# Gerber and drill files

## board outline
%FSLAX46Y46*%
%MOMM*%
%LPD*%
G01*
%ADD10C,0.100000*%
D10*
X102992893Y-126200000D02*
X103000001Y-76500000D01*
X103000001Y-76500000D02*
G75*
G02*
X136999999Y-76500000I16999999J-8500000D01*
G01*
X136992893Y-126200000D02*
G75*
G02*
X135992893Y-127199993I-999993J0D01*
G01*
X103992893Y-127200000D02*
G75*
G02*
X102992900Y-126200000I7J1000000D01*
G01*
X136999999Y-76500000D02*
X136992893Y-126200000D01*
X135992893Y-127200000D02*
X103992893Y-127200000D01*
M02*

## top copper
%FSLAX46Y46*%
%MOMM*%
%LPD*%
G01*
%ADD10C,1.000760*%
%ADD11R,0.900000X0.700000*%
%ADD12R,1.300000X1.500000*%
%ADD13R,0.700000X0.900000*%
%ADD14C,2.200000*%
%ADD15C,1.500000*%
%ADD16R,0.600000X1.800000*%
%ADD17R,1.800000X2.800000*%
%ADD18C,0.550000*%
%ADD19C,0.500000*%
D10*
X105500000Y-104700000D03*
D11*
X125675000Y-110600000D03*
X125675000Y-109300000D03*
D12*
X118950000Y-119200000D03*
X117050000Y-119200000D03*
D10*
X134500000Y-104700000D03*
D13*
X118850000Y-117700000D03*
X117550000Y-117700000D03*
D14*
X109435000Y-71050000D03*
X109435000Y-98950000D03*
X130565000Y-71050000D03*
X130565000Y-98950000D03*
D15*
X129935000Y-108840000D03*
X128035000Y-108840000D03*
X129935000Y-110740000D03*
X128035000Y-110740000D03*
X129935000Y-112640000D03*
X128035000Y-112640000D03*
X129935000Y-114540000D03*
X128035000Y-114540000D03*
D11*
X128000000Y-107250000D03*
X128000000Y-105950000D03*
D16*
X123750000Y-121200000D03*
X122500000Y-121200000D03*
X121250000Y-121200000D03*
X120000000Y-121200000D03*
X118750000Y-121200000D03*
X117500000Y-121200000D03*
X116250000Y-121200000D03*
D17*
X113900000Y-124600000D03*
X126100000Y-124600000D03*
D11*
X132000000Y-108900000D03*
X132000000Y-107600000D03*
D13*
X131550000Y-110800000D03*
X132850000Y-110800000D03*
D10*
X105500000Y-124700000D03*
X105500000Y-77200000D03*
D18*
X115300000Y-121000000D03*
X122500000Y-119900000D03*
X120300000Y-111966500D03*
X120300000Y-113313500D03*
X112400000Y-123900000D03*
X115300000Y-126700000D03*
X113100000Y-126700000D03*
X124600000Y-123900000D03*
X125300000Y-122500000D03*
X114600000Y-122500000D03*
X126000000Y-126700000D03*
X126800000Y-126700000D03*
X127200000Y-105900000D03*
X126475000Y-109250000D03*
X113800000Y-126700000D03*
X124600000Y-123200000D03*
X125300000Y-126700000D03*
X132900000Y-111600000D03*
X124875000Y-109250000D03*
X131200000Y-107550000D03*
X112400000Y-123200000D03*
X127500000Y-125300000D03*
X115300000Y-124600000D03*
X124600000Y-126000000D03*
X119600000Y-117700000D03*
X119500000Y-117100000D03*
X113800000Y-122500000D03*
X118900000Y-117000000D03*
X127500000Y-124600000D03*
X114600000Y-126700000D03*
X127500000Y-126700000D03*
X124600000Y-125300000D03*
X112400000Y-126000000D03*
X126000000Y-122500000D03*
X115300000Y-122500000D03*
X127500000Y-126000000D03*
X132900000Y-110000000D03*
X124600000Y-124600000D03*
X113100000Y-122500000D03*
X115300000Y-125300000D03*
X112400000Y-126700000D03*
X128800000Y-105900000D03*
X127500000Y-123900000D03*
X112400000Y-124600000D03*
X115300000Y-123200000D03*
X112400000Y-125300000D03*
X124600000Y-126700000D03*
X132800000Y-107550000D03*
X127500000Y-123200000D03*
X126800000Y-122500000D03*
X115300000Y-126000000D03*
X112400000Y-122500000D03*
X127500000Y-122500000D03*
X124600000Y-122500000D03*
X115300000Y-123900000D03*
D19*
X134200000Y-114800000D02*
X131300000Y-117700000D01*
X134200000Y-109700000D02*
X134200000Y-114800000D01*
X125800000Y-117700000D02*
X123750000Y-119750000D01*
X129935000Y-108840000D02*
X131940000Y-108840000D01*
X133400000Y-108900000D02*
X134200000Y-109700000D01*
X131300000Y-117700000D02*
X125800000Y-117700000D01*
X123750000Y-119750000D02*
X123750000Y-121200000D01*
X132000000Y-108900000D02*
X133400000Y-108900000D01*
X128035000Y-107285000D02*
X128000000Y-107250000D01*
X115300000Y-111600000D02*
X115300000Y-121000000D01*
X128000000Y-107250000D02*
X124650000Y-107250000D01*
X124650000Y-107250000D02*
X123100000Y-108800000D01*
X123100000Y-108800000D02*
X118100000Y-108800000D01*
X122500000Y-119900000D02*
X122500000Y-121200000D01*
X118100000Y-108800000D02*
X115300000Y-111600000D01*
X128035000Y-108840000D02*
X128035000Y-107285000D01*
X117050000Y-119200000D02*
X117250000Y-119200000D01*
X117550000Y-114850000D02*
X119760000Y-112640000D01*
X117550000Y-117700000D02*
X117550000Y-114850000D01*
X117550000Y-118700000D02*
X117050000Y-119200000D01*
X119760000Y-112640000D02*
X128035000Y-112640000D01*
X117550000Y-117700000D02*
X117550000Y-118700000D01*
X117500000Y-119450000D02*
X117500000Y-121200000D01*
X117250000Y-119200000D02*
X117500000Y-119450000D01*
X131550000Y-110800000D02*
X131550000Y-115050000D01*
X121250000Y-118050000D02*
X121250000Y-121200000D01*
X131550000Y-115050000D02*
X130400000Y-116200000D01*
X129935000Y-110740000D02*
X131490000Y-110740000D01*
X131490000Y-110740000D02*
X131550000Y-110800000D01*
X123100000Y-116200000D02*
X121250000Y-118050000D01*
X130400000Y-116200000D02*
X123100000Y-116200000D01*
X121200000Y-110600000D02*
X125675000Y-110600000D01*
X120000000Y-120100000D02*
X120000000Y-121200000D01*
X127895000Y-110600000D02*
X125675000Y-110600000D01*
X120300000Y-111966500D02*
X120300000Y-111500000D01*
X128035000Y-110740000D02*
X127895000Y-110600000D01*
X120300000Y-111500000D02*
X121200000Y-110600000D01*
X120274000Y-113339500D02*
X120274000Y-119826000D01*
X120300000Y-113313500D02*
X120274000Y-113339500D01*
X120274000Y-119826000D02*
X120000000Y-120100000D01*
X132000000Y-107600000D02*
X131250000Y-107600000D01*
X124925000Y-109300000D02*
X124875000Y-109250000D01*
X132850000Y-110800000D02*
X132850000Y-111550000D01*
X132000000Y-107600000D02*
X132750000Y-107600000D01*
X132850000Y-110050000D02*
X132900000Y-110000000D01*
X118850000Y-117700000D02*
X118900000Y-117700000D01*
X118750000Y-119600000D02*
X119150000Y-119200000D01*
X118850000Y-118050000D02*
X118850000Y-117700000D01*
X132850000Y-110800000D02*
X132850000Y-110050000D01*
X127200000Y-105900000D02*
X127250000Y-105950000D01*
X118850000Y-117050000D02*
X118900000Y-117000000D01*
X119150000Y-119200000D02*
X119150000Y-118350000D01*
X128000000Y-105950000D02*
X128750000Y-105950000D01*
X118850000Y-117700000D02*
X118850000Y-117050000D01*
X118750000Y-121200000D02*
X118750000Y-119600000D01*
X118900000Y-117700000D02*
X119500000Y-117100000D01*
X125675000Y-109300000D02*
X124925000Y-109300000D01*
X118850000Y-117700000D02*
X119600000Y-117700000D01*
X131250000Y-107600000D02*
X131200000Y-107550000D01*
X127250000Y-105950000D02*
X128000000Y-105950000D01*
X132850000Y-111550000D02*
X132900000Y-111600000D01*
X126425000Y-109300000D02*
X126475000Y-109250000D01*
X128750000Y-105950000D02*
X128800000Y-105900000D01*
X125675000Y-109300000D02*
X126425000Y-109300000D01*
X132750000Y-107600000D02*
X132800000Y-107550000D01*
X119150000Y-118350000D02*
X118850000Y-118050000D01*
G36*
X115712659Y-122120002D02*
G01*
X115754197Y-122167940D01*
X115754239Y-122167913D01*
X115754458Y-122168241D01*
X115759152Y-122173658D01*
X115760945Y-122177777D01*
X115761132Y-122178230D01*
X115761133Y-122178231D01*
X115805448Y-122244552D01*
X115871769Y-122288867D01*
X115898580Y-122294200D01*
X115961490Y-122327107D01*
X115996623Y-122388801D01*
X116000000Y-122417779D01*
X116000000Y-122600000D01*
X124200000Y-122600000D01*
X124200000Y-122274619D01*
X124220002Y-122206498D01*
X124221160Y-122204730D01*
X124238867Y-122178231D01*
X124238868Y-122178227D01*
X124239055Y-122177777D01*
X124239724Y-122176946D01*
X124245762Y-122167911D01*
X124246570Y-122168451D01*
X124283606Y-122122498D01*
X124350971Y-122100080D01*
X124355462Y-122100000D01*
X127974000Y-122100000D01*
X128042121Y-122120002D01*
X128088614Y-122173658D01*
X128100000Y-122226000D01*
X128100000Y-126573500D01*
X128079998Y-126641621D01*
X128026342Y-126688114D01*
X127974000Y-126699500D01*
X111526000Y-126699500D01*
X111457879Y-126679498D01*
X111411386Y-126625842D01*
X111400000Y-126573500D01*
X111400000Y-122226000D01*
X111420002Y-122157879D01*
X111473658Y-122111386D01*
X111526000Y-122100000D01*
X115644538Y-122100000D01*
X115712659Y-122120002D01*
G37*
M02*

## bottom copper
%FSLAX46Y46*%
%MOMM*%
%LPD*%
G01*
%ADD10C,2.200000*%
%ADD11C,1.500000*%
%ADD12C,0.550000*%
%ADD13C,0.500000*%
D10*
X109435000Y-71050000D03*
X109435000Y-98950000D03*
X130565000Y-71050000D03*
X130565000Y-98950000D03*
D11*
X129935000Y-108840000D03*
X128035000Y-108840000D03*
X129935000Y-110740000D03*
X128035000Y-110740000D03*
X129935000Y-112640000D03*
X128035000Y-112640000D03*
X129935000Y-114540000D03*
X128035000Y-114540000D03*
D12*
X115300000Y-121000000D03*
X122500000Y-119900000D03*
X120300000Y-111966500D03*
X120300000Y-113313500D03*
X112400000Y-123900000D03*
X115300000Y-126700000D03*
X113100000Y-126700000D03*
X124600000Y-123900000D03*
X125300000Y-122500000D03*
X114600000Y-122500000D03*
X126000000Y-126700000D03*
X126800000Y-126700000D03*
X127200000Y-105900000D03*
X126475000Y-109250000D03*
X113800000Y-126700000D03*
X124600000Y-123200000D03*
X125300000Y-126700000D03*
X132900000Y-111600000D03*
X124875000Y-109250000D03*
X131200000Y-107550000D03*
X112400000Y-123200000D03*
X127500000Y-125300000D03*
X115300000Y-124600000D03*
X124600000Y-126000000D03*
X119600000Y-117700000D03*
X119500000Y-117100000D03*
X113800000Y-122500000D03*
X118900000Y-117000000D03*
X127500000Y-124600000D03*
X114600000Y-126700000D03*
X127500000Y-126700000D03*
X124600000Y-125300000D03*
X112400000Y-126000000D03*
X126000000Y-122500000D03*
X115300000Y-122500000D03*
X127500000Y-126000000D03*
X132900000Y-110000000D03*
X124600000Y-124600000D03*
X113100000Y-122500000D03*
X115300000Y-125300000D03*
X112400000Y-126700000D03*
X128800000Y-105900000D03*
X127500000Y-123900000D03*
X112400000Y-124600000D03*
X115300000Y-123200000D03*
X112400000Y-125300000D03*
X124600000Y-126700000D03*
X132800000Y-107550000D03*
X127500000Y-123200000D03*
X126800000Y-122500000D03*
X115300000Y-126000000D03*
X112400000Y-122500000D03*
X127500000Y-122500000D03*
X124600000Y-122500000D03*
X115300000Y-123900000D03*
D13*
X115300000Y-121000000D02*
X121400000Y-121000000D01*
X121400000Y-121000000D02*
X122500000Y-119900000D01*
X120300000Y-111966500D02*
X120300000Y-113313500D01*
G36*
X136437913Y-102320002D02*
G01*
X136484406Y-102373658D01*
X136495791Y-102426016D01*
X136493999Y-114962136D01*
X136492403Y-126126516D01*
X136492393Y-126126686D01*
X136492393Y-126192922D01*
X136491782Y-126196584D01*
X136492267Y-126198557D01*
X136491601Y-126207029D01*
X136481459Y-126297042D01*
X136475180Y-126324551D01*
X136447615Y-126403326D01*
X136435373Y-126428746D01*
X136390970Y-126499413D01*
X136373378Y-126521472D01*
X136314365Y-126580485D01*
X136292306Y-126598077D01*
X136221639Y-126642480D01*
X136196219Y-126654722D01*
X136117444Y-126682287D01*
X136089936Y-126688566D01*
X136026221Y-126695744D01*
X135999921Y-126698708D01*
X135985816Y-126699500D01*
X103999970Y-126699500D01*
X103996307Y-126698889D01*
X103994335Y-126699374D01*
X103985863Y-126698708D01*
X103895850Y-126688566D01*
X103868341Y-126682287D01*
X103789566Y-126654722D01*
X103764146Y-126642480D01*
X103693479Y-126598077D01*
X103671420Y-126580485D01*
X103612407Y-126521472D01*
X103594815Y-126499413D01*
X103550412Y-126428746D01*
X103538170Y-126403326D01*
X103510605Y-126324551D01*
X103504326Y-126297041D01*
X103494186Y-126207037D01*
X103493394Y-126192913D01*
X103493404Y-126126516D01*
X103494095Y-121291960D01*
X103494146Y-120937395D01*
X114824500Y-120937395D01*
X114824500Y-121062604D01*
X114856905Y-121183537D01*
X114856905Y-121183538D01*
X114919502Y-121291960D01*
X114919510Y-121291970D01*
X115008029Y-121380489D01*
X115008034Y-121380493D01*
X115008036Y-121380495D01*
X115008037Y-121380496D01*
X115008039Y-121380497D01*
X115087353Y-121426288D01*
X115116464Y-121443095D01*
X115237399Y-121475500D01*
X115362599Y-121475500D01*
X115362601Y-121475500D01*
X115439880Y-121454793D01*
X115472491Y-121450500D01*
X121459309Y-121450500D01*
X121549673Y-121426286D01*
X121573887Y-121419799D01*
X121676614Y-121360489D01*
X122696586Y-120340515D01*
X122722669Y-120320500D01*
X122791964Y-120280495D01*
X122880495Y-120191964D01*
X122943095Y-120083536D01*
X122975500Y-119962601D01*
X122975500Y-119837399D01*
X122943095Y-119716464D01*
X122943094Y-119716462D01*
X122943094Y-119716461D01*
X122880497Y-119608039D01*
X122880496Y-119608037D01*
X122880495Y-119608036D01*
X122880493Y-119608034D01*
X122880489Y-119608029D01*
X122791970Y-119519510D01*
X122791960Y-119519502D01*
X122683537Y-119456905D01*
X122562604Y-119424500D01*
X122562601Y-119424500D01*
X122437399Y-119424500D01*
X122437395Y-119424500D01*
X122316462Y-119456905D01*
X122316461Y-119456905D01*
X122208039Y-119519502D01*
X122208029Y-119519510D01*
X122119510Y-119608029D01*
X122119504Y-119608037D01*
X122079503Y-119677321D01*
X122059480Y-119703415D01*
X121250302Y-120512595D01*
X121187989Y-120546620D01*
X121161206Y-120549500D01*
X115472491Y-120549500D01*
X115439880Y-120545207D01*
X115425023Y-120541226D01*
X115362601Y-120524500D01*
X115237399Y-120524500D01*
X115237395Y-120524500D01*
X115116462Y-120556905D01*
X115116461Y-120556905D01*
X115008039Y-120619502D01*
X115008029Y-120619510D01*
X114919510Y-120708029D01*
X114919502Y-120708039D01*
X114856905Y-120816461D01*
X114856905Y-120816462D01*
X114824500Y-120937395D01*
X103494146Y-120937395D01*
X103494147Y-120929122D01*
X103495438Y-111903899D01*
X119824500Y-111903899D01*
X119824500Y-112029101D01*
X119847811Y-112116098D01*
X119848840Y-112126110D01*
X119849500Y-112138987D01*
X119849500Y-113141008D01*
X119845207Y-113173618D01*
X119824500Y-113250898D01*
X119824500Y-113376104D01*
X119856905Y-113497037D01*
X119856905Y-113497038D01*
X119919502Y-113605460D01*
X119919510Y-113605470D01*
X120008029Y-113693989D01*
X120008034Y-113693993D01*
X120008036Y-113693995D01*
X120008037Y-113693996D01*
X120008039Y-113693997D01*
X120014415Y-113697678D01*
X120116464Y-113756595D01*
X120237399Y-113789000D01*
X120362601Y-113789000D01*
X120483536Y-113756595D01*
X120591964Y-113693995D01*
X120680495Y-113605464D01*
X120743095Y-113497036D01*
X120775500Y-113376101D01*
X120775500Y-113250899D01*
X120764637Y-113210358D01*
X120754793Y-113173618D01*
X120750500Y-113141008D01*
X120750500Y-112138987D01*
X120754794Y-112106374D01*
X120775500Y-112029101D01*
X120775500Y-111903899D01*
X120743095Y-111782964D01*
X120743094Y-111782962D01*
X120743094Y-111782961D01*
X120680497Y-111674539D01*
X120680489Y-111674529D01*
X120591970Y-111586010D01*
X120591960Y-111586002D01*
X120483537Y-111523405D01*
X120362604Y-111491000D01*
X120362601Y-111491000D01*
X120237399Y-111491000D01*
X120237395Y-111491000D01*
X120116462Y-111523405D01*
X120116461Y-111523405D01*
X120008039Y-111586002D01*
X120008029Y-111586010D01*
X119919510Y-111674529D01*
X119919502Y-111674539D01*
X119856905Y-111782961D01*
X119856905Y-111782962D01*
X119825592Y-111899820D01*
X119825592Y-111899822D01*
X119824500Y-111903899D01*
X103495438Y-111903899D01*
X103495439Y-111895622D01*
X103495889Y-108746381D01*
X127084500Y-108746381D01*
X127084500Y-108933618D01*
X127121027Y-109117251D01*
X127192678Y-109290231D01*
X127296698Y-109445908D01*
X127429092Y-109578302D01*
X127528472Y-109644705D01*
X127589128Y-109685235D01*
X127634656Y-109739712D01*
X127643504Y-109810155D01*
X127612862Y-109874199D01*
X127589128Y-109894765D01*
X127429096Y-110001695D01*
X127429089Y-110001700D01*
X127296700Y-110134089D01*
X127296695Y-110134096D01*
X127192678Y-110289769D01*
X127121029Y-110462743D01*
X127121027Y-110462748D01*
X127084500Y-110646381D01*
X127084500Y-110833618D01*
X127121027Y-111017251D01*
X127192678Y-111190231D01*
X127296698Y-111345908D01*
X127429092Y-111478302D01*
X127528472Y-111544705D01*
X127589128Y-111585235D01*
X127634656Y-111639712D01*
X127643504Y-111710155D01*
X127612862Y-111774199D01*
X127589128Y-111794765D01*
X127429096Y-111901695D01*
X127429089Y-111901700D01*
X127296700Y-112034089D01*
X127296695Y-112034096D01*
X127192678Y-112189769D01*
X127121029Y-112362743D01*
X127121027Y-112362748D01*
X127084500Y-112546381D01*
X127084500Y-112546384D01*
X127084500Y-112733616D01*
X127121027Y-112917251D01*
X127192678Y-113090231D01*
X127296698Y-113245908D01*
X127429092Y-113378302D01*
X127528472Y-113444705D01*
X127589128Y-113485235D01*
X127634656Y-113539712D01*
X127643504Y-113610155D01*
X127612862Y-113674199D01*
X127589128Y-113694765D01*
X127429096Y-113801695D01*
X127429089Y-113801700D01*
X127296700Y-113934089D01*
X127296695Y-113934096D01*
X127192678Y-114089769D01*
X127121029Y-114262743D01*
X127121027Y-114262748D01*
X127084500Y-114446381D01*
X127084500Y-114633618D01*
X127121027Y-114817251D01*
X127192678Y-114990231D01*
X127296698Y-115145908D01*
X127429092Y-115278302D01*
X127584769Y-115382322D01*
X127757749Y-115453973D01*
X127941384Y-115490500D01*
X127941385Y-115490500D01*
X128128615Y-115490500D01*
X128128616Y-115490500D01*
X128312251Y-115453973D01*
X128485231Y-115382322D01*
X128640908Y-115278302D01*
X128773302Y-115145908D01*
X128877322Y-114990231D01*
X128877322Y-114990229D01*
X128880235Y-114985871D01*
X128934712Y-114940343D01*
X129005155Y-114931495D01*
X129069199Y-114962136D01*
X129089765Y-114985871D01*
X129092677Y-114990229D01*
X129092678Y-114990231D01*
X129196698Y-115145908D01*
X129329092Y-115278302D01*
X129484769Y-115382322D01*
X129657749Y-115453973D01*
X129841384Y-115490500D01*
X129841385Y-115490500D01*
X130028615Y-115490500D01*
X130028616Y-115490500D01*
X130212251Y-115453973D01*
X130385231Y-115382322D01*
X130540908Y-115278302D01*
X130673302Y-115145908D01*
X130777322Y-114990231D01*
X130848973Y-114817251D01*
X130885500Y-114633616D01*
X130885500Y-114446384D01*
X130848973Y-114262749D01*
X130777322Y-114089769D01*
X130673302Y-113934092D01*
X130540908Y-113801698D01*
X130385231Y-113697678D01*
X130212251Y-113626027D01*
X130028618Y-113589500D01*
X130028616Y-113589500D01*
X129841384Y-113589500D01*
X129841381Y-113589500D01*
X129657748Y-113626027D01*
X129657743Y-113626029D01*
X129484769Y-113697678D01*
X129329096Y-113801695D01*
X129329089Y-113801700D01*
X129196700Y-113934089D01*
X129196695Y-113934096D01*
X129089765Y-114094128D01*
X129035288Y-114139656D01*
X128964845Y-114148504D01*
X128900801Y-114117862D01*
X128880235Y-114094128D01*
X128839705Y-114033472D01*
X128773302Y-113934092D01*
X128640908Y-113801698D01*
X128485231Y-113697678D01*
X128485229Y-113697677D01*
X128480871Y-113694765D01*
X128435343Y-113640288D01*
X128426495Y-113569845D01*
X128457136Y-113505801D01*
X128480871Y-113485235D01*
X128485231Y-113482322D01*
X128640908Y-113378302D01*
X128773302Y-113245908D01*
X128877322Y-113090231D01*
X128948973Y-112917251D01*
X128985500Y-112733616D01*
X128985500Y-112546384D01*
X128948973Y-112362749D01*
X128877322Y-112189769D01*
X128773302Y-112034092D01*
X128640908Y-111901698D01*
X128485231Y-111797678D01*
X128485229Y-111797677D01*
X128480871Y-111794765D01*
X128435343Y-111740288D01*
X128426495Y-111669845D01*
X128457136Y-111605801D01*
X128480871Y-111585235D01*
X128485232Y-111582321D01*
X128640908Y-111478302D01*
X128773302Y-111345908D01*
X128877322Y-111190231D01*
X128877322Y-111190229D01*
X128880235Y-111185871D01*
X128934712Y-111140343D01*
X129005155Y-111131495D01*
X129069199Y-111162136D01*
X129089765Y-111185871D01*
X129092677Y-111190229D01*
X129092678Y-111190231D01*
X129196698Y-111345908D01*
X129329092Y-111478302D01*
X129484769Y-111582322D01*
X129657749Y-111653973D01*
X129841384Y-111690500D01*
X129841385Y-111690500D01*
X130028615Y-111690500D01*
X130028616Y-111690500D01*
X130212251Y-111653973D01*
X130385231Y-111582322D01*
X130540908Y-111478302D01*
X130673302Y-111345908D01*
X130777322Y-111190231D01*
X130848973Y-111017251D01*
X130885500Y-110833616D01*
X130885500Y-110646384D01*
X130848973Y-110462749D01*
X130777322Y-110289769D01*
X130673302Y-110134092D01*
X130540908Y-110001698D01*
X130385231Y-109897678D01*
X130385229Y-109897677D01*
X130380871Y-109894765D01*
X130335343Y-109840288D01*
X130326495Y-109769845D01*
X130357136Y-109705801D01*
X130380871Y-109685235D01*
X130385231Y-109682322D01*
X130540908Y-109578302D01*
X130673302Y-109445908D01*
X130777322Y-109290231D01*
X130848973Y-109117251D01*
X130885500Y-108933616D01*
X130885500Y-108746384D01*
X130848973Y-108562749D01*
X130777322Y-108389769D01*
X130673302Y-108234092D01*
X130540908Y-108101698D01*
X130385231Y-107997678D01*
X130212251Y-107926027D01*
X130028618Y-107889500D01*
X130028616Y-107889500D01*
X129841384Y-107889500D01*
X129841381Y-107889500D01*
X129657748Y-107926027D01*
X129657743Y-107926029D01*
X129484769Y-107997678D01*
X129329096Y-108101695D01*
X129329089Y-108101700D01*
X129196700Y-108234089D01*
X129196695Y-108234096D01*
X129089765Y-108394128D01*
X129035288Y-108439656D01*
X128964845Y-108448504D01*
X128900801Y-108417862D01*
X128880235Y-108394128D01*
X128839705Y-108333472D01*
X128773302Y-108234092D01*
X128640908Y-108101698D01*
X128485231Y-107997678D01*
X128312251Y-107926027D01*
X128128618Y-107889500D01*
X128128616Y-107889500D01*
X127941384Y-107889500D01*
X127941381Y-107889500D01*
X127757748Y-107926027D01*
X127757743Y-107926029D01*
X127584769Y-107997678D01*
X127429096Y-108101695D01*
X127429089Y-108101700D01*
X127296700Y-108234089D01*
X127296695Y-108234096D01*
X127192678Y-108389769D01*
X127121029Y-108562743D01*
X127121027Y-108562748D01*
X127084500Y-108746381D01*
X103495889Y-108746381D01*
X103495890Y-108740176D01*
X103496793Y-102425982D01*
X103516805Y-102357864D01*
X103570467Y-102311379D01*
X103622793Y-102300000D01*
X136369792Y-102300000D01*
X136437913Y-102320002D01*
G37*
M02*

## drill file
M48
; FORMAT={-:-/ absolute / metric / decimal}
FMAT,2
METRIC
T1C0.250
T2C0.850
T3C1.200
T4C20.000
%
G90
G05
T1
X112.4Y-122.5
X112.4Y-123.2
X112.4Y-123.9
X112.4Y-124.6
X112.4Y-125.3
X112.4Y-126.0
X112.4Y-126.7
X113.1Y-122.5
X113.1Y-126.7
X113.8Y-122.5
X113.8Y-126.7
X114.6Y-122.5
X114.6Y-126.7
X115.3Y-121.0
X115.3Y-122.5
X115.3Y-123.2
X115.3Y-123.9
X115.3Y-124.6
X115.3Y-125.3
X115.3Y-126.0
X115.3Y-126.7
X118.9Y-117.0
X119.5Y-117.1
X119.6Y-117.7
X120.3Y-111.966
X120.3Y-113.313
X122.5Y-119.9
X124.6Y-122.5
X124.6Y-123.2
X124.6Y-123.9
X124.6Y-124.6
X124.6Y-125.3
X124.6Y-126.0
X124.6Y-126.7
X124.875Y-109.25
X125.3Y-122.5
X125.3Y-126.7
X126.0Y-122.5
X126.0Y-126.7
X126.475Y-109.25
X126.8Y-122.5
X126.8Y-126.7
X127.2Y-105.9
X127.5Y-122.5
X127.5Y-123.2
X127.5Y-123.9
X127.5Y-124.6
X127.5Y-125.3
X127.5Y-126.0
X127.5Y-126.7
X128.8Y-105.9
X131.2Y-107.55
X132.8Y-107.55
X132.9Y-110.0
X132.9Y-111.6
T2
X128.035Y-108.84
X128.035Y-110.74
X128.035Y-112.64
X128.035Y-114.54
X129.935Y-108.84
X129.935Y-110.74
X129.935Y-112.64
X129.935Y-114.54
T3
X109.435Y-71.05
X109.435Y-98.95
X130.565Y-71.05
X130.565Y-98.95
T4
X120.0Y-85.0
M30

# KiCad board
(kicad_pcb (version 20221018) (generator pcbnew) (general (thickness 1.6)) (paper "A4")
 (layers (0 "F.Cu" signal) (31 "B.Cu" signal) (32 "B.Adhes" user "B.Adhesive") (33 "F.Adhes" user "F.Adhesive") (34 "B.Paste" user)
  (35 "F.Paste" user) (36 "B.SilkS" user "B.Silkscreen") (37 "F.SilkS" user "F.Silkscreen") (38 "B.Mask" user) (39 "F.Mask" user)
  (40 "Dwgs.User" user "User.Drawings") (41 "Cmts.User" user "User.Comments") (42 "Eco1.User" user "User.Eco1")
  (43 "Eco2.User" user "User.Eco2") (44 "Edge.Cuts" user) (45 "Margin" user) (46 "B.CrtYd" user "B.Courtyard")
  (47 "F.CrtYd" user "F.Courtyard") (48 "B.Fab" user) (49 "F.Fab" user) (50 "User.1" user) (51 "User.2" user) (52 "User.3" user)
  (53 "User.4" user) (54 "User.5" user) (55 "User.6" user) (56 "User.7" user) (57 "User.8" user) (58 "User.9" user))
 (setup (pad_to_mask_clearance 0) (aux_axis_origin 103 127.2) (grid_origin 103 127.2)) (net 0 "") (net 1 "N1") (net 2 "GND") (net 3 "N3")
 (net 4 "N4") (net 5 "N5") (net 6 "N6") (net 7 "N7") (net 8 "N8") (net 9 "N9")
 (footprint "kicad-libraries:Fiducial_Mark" (layer "F.Cu") (at 105.5 104.7)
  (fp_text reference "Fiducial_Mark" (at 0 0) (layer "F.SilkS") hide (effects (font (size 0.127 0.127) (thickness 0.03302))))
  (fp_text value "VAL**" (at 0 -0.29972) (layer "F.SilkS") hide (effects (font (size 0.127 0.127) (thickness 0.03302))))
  (pad "1" smd circle (at 0 0) (size 1.00076 1.00076) (layers "F.Cu" "F.Paste" "F.Mask") (clearance 0.65024)))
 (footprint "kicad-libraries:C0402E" (layer "F.Cu") (at 125.675 109.95 90)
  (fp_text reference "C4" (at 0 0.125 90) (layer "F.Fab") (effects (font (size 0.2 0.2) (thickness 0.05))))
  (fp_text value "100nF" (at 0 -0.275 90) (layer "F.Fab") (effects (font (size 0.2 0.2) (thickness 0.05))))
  (pad "1" smd rect (at -0.65 0 90) (size 0.7 0.9) (layers "F.Cu" "F.Paste" "F.Mask") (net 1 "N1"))
  (pad "2" smd rect (at 0.65 0 90) (size 0.7 0.9) (layers "F.Cu" "F.Paste" "F.Mask") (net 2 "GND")))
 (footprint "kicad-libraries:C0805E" (layer "F.Cu") (at 118 119.2 180)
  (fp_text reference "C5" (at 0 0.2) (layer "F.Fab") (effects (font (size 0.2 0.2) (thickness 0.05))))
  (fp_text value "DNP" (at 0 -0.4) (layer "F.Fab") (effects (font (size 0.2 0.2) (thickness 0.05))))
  (pad "1" smd rect (at -0.95 0 180) (size 1.3 1.5) (layers "F.Cu" "F.Paste" "F.Mask") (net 2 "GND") (clearance 0.14986))
  (pad "2" smd rect (at 0.95 0 180) (size 1.3 1.5) (layers "F.Cu" "F.Paste" "F.Mask") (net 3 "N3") (clearance 0.14986)))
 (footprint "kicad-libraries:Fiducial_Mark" (layer "F.Cu") (at 134.5 104.7)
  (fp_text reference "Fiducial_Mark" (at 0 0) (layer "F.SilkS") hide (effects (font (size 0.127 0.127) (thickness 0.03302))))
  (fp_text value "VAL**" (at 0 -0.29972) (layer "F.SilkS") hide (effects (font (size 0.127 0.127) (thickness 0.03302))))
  (pad "1" smd circle (at 0 0) (size 1.00076 1.00076) (layers "F.Cu" "F.Paste" "F.Mask") (clearance 0.65024)))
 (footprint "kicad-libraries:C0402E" (layer "F.Cu") (at 118.2 117.7 180)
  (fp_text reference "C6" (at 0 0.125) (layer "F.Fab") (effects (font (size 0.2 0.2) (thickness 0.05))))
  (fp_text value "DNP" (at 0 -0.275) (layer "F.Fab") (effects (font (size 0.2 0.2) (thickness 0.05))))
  (pad "1" smd rect (at -0.65 0 180) (size 0.7 0.9) (layers "F.Cu" "F.Paste" "F.Mask") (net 2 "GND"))
  (pad "2" smd rect (at 0.65 0 180) (size 0.7 0.9) (layers "F.Cu" "F.Paste" "F.Mask") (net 3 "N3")))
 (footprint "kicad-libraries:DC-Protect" (layer "F.Cu") (at 120 85)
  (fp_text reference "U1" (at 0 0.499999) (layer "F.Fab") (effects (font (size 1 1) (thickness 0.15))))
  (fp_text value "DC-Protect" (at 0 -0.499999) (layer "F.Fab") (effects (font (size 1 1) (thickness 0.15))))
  (pad "" thru_hole circle (at -10.565 -13.95) (size 2.2 2.2) (drill 1.2) (layers "F&B.Cu" "*.Mask"))
  (pad "" thru_hole circle (at -10.565 13.95) (size 2.2 2.2) (drill 1.2) (layers "F&B.Cu" "*.Mask"))
  (pad "" np_thru_hole circle (at 0 0) (size 20 20) (drill 20) (layers "F&B.Cu" "*.Mask"))
  (pad "" thru_hole circle (at 10.565 -13.95) (size 2.2 2.2) (drill 1.2) (layers "F&B.Cu" "*.Mask"))
  (pad "" thru_hole circle (at 10.565 13.95) (size 2.2 2.2) (drill 1.2) (layers "F&B.Cu" "*.Mask"))
  (pad "1" thru_hole circle (at 9.935 23.84) (size 1.5 1.5) (drill 0.85) (layers "F&B.Cu" "*.Mask") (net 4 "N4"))
  (pad "2" thru_hole circle (at 8.035 23.84) (size 1.5 1.5) (drill 0.85) (layers "F&B.Cu" "*.Mask") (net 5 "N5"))
  (pad "3" thru_hole circle (at 9.935 25.74) (size 1.5 1.5) (drill 0.85) (layers "F&B.Cu" "*.Mask") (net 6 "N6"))
  (pad "4" thru_hole circle (at 8.035 25.74) (size 1.5 1.5) (drill 0.85) (layers "F&B.Cu" "*.Mask") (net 1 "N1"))
  (pad "5" thru_hole circle (at 9.935 27.64) (size 1.5 1.5) (drill 0.85) (layers "F&B.Cu" "*.Mask") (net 2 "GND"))
  (pad "6" thru_hole circle (at 8.035 27.64) (size 1.5 1.5) (drill 0.85) (layers "F&B.Cu" "*.Mask") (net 3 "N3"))
  (pad "7" thru_hole circle (at 9.935 29.54) (size 1.5 1.5) (drill 0.85) (layers "F&B.Cu" "*.Mask") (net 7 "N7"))
  (pad "8" thru_hole circle (at 8.035 29.54) (size 1.5 1.5) (drill 0.85) (layers "F&B.Cu" "*.Mask") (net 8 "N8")))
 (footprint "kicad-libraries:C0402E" (layer "F.Cu") (at 128 106.6 90)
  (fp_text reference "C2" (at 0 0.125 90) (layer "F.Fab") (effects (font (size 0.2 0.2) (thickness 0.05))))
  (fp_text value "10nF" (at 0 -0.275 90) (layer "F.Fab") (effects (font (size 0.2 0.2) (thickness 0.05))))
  (pad "1" smd rect (at -0.65 0 90) (size 0.7 0.9) (layers "F.Cu" "F.Paste" "F.Mask") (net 5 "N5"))
  (pad "2" smd rect (at 0.65 0 90) (size 0.7 0.9) (layers "F.Cu" "F.Paste" "F.Mask") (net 2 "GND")))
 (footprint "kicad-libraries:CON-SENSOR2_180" (layer "F.Cu") (at 120 126)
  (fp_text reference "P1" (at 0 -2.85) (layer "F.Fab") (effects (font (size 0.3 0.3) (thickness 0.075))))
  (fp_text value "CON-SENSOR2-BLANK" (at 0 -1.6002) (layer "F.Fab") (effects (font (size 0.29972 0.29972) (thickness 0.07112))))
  (pad "1" smd rect (at 3.75 -4.8) (size 0.6 1.8) (layers "F.Cu" "F.Paste" "F.Mask") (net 4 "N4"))
  (pad "2" smd rect (at 2.5 -4.8) (size 0.6 1.8) (layers "F.Cu" "F.Paste" "F.Mask") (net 5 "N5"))
  (pad "3" smd rect (at 1.25 -4.8) (size 0.6 1.8) (layers "F.Cu" "F.Paste" "F.Mask") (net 6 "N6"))
  (pad "4" smd rect (at 0 -4.8) (size 0.6 1.8) (layers "F.Cu" "F.Paste" "F.Mask") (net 1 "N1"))
  (pad "5" smd rect (at -1.25 -4.8) (size 0.6 1.8) (layers "F.Cu" "F.Paste" "F.Mask") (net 2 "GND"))
  (pad "6" smd rect (at -2.5 -4.8) (size 0.6 1.8) (layers "F.Cu" "F.Paste" "F.Mask") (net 3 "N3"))
  (pad "7" smd rect (at -3.75 -4.8) (size 0.6 1.8) (layers "F.Cu" "F.Paste" "F.Mask") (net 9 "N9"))
  (pad "EP" smd rect (at -6.1 -1.4) (size 1.8 2.8) (layers "F.Cu" "F.Paste" "F.Mask") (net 2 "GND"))
  (pad "EP" smd rect (at 6.1 -1.4) (size 1.8 2.8) (layers "F.Cu" "F.Paste" "F.Mask") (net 2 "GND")))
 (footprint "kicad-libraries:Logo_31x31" (layer "F.Cu") (at 109 122.9 180)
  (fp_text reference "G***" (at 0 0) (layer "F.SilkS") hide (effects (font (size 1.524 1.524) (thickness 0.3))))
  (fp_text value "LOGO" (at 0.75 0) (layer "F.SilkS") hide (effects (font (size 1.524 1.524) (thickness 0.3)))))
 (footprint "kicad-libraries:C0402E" (layer "F.Cu") (at 132 108.25 90)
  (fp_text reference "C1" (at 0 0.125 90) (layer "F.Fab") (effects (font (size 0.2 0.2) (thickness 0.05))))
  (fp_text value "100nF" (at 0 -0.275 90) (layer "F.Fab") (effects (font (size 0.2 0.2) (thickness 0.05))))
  (pad "1" smd rect (at -0.65 0 90) (size 0.7 0.9) (layers "F.Cu" "F.Paste" "F.Mask") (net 4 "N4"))
  (pad "2" smd rect (at 0.65 0 90) (size 0.7 0.9) (layers "F.Cu" "F.Paste" "F.Mask") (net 2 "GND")))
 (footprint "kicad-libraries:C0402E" (layer "F.Cu") (at 132.2 110.8)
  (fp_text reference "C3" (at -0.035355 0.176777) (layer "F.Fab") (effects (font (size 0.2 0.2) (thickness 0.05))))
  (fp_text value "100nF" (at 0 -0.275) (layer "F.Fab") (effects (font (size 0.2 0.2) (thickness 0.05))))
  (pad "1" smd rect (at -0.65 0) (size 0.7 0.9) (layers "F.Cu" "F.Paste" "F.Mask") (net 6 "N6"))
  (pad "2" smd rect (at 0.65 0) (size 0.7 0.9) (layers "F.Cu" "F.Paste" "F.Mask") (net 2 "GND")))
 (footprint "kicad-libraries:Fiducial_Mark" (layer "F.Cu") (at 105.5 124.7)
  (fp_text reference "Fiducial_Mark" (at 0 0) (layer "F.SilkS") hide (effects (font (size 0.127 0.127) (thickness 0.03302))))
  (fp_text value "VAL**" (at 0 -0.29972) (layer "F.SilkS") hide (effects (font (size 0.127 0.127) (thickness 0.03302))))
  (pad "1" smd circle (at 0 0) (size 1.00076 1.00076) (layers "F.Cu" "F.Paste" "F.Mask") (clearance 0.65024)))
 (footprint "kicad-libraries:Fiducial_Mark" (layer "F.Cu") (at 105.5 77.2)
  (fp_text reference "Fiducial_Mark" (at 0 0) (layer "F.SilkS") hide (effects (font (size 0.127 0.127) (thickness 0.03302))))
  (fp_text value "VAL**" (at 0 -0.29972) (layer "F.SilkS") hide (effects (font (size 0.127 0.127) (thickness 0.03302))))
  (pad "1" smd circle (at 0 0) (size 1.00076 1.00076) (layers "F.Cu" "F.Paste" "F.Mask") (clearance 0.65024)))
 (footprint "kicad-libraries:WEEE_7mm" (layer "F.Cu") (at 133 122.1 180)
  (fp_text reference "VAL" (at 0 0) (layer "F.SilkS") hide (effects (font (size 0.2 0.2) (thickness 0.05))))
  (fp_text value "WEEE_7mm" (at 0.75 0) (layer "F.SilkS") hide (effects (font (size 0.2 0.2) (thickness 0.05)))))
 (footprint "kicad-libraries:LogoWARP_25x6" (layer "B.Cu") (at 120 123)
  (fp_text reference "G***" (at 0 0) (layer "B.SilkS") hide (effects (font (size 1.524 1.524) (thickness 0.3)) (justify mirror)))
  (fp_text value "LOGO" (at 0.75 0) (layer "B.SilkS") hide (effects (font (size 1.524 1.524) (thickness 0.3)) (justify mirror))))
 (gr_line (start 102.992893 126.2) (end 103.000001 76.5) (stroke (width 0.1) (type solid)) (layer "Edge.Cuts"))
 (gr_arc (start 103.000001 76.5) (mid 120 65.993423) (end 136.999999 76.5) (stroke (width 0.1) (type solid)) (layer "Edge.Cuts"))
 (gr_arc (start 136.992893 126.2) (mid 136.7 126.907107) (end 135.992893 127.2) (stroke (width 0.1) (type solid)) (layer "Edge.Cuts"))
 (gr_arc (start 103.992893 127.2) (mid 103.285786 126.907107) (end 102.992893 126.2) (stroke (width 0.1) (type solid)) (layer "Edge.Cuts"))
 (gr_line (start 136.999999 76.5) (end 136.992893 126.2) (stroke (width 0.1) (type solid)) (layer "Edge.Cuts"))
 (gr_line (start 135.992893 127.2) (end 103.992893 127.2) (stroke (width 0.1) (type solid)) (layer "Edge.Cuts"))
 (segment (start 134.2 114.8) (end 131.3 117.7) (width 0.5) (layer "F.Cu") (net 4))
 (segment (start 134.2 109.7) (end 134.2 114.8) (width 0.5) (layer "F.Cu") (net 4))
 (segment (start 125.8 117.7) (end 123.75 119.75) (width 0.5) (layer "F.Cu") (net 4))
 (segment (start 129.935 108.84) (end 131.94 108.84) (width 0.5) (layer "F.Cu") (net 4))
 (segment (start 133.4 108.9) (end 134.2 109.7) (width 0.5) (layer "F.Cu") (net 4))
 (segment (start 131.3 117.7) (end 125.8 117.7) (width 0.5) (layer "F.Cu") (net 4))
 (segment (start 123.75 119.75) (end 123.75 121.2) (width 0.5) (layer "F.Cu") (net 4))
 (segment (start 132 108.9) (end 133.4 108.9) (width 0.5) (layer "F.Cu") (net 4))
 (segment (start 128.035 107.285) (end 128 107.25) (width 0.5) (layer "F.Cu") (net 5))
 (segment (start 115.3 111.6) (end 115.3 121) (width 0.5) (layer "F.Cu") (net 5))
 (segment (start 128 107.25) (end 124.65 107.25) (width 0.5) (layer "F.Cu") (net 5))
 (segment (start 124.65 107.25) (end 123.1 108.8) (width 0.5) (layer "F.Cu") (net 5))
 (segment (start 123.1 108.8) (end 118.1 108.8) (width 0.5) (layer "F.Cu") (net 5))
 (segment (start 122.5 119.9) (end 122.5 121.2) (width 0.5) (layer "F.Cu") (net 5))
 (segment (start 118.1 108.8) (end 115.3 111.6) (width 0.5) (layer "F.Cu") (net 5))
 (segment (start 128.035 108.84) (end 128.035 107.285) (width 0.5) (layer "F.Cu") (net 5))
 (via (at 115.3 121) (size 0.55) (drill 0.25) (layers "F.Cu" "B.Cu") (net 5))
 (via (at 122.5 119.9) (size 0.55) (drill 0.25) (layers "F.Cu" "B.Cu") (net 5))
 (segment (start 115.3 121) (end 121.4 121) (width 0.5) (layer "B.Cu") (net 5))
 (segment (start 121.4 121) (end 122.5 119.9) (width 0.5) (layer "B.Cu") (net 5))
 (segment (start 117.05 119.2) (end 117.25 119.2) (width 0.5) (layer "F.Cu") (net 3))
 (segment (start 117.55 114.85) (end 119.76 112.64) (width 0.5) (layer "F.Cu") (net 3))
 (segment (start 117.55 117.7) (end 117.55 114.85) (width 0.5) (layer "F.Cu") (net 3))
 (segment (start 117.55 118.7) (end 117.05 119.2) (width 0.5) (layer "F.Cu") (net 3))
 (segment (start 119.76 112.64) (end 128.035 112.64) (width 0.5) (layer "F.Cu") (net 3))
 (segment (start 117.55 117.7) (end 117.55 118.7) (width 0.5) (layer "F.Cu") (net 3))
 (segment (start 117.5 119.45) (end 117.5 121.2) (width 0.5) (layer "F.Cu") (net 3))
 (segment (start 117.25 119.2) (end 117.5 119.45) (width 0.5) (layer "F.Cu") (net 3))
 (segment (start 131.55 110.8) (end 131.55 115.05) (width 0.5) (layer "F.Cu") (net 6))
 (segment (start 121.25 118.05) (end 121.25 121.2) (width 0.5) (layer "F.Cu") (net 6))
 (segment (start 131.55 115.05) (end 130.4 116.2) (width 0.5) (layer "F.Cu") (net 6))
 (segment (start 129.935 110.74) (end 131.49 110.74) (width 0.5) (layer "F.Cu") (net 6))
 (segment (start 131.49 110.74) (end 131.55 110.8) (width 0.5) (layer "F.Cu") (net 6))
 (segment (start 123.1 116.2) (end 121.25 118.05) (width 0.5) (layer "F.Cu") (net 6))
 (segment (start 130.4 116.2) (end 123.1 116.2) (width 0.5) (layer "F.Cu") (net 6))
 (segment (start 121.2 110.6) (end 125.675 110.6) (width 0.5) (layer "F.Cu") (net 1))
 (segment (start 120 120.1) (end 120 121.2) (width 0.5) (layer "F.Cu") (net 1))
 (segment (start 127.895 110.6) (end 125.675 110.6) (width 0.5) (layer "F.Cu") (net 1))
 (segment (start 120.3 111.9665) (end 120.3 111.5) (width 0.5) (layer "F.Cu") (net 1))
 (segment (start 128.035 110.74) (end 127.895 110.6) (width 0.5) (layer "F.Cu") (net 1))
 (segment (start 120.3 111.5) (end 121.2 110.6) (width 0.5) (layer "F.Cu") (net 1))
 (segment (start 120.274 113.3395) (end 120.274 119.826) (width 0.5) (layer "F.Cu") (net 1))
 (segment (start 120.3 113.3135) (end 120.274 113.3395) (width 0.5) (layer "F.Cu") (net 1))
 (segment (start 120.274 119.826) (end 120 120.1) (width 0.5) (layer "F.Cu") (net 1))
 (via (at 120.3 111.9665) (size 0.55) (drill 0.25) (layers "F.Cu" "B.Cu") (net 1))
 (via (at 120.3 113.3135) (size 0.55) (drill 0.25) (layers "F.Cu" "B.Cu") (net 1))
 (segment (start 120.3 111.9665) (end 120.3 113.3135) (width 0.5) (layer "B.Cu") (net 1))
 (segment (start 132 107.6) (end 131.25 107.6) (width 0.5) (layer "F.Cu") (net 2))
 (segment (start 124.925 109.3) (end 124.875 109.25) (width 0.5) (layer "F.Cu") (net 2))
 (segment (start 132.85 110.8) (end 132.85 111.55) (width 0.5) (layer "F.Cu") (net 2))
 (segment (start 132 107.6) (end 132.75 107.6) (width 0.5) (layer "F.Cu") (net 2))
 (segment (start 132.85 110.05) (end 132.9 110) (width 0.5) (layer "F.Cu") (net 2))
 (segment (start 118.85 117.7) (end 118.9 117.7) (width 0.5) (layer "F.Cu") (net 2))
 (segment (start 118.75 119.6) (end 119.15 119.2) (width 0.5) (layer "F.Cu") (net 2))
 (segment (start 118.85 118.05) (end 118.85 117.7) (width 0.5) (layer "F.Cu") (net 2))
 (segment (start 132.85 110.8) (end 132.85 110.05) (width 0.5) (layer "F.Cu") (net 2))
 (segment (start 127.2 105.9) (end 127.25 105.95) (width 0.5) (layer "F.Cu") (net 2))
 (segment (start 118.85 117.05) (end 118.9 117) (width 0.5) (layer "F.Cu") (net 2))
 (segment (start 119.15 119.2) (end 119.15 118.35) (width 0.5) (layer "F.Cu") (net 2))
 (segment (start 128 105.95) (end 128.75 105.95) (width 0.5) (layer "F.Cu") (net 2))
 (segment (start 118.85 117.7) (end 118.85 117.05) (width 0.5) (layer "F.Cu") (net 2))
 (segment (start 118.75 121.2) (end 118.75 119.6) (width 0.5) (layer "F.Cu") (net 2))
 (segment (start 118.9 117.7) (end 119.5 117.1) (width 0.5) (layer "F.Cu") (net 2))
 (segment (start 125.675 109.3) (end 124.925 109.3) (width 0.5) (layer "F.Cu") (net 2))
 (segment (start 118.85 117.7) (end 119.6 117.7) (width 0.5) (layer "F.Cu") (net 2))
 (segment (start 131.25 107.6) (end 131.2 107.55) (width 0.5) (layer "F.Cu") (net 2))
 (segment (start 127.25 105.95) (end 128 105.95) (width 0.5) (layer "F.Cu") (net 2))
 (segment (start 132.85 111.55) (end 132.9 111.6) (width 0.5) (layer "F.Cu") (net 2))
 (segment (start 126.425 109.3) (end 126.475 109.25) (width 0.5) (layer "F.Cu") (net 2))
 (segment (start 128.75 105.95) (end 128.8 105.9) (width 0.5) (layer "F.Cu") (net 2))
 (segment (start 125.675 109.3) (end 126.425 109.3) (width 0.5) (layer "F.Cu") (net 2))
 (segment (start 132.75 107.6) (end 132.8 107.55) (width 0.5) (layer "F.Cu") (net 2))
 (segment (start 119.15 118.35) (end 118.85 118.05) (width 0.5) (layer "F.Cu") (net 2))
 (via (at 112.4 123.9) (size 0.55) (drill 0.25) (layers "F.Cu" "B.Cu") (free) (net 2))
 (via (at 115.3 126.7) (size 0.55) (drill 0.25) (layers "F.Cu" "B.Cu") (free) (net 2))
 (via (at 113.1 126.7) (size 0.55) (drill 0.25) (layers "F.Cu" "B.Cu") (free) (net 2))
 (via (at 124.6 123.9) (size 0.55) (drill 0.25) (layers "F.Cu" "B.Cu") (free) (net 2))
 (via (at 125.3 122.5) (size 0.55) (drill 0.25) (layers "F.Cu" "B.Cu") (free) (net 2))
 (via (at 114.6 122.5) (size 0.55) (drill 0.25) (layers "F.Cu" "B.Cu") (free) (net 2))
 (via (at 126 126.7) (size 0.55) (drill 0.25) (layers "F.Cu" "B.Cu") (free) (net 2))
 (via (at 126.8 126.7) (size 0.55) (drill 0.25) (layers "F.Cu" "B.Cu") (free) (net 2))
 (via (at 127.2 105.9) (size 0.55) (drill 0.25) (layers "F.Cu" "B.Cu") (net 2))
 (via (at 126.475 109.25) (size 0.55) (drill 0.25) (layers "F.Cu" "B.Cu") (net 2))
 (via (at 113.8 126.7) (size 0.55) (drill 0.25) (layers "F.Cu" "B.Cu") (free) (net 2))
 (via (at 124.6 123.2) (size 0.55) (drill 0.25) (layers "F.Cu" "B.Cu") (free) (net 2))
 (via (at 125.3 126.7) (size 0.55) (drill 0.25) (layers "F.Cu" "B.Cu") (free) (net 2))
 (via (at 132.9 111.6) (size 0.55) (drill 0.25) (layers "F.Cu" "B.Cu") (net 2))
 (via (at 124.875 109.25) (size 0.55) (drill 0.25) (layers "F.Cu" "B.Cu") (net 2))
 (via (at 131.2 107.55) (size 0.55) (drill 0.25) (layers "F.Cu" "B.Cu") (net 2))
 (via (at 112.4 123.2) (size 0.55) (drill 0.25) (layers "F.Cu" "B.Cu") (free) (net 2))
 (via (at 127.5 125.3) (size 0.55) (drill 0.25) (layers "F.Cu" "B.Cu") (free) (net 2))
 (via (at 115.3 124.6) (size 0.55) (drill 0.25) (layers "F.Cu" "B.Cu") (free) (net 2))
 (via (at 124.6 126) (size 0.55) (drill 0.25) (layers "F.Cu" "B.Cu") (free) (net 2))
 (via (at 119.6 117.7) (size 0.55) (drill 0.25) (layers "F.Cu" "B.Cu") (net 2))
 (via (at 119.5 117.1) (size 0.55) (drill 0.25) (layers "F.Cu" "B.Cu") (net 2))
 (via (at 113.8 122.5) (size 0.55) (drill 0.25) (layers "F.Cu" "B.Cu") (free) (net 2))
 (via (at 118.9 117) (size 0.55) (drill 0.25) (layers "F.Cu" "B.Cu") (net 2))
 (via (at 127.5 124.6) (size 0.55) (drill 0.25) (layers "F.Cu" "B.Cu") (free) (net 2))
 (via (at 114.6 126.7) (size 0.55) (drill 0.25) (layers "F.Cu" "B.Cu") (free) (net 2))
 (via (at 127.5 126.7) (size 0.55) (drill 0.25) (layers "F.Cu" "B.Cu") (free) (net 2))
 (via (at 124.6 125.3) (size 0.55) (drill 0.25) (layers "F.Cu" "B.Cu") (free) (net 2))
 (via (at 112.4 126) (size 0.55) (drill 0.25) (layers "F.Cu" "B.Cu") (free) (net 2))
 (via (at 126 122.5) (size 0.55) (drill 0.25) (layers "F.Cu" "B.Cu") (free) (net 2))
 (via (at 115.3 122.5) (size 0.55) (drill 0.25) (layers "F.Cu" "B.Cu") (free) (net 2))
 (via (at 127.5 126) (size 0.55) (drill 0.25) (layers "F.Cu" "B.Cu") (free) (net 2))
 (via (at 132.9 110) (size 0.55) (drill 0.25) (layers "F.Cu" "B.Cu") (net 2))
 (via (at 124.6 124.6) (size 0.55) (drill 0.25) (layers "F.Cu" "B.Cu") (free) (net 2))
 (via (at 113.1 122.5) (size 0.55) (drill 0.25) (layers "F.Cu" "B.Cu") (free) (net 2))
 (via (at 115.3 125.3) (size 0.55) (drill 0.25) (layers "F.Cu" "B.Cu") (free) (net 2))
 (via (at 112.4 126.7) (size 0.55) (drill 0.25) (layers "F.Cu" "B.Cu") (free) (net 2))
 (via (at 128.8 105.9) (size 0.55) (drill 0.25) (layers "F.Cu" "B.Cu") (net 2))
 (via (at 127.5 123.9) (size 0.55) (drill 0.25) (layers "F.Cu" "B.Cu") (free) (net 2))
 (via (at 112.4 124.6) (size 0.55) (drill 0.25) (layers "F.Cu" "B.Cu") (free) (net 2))
 (via (at 115.3 123.2) (size 0.55) (drill 0.25) (layers "F.Cu" "B.Cu") (free) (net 2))
 (via (at 112.4 125.3) (size 0.55) (drill 0.25) (layers "F.Cu" "B.Cu") (free) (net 2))
 (via (at 124.6 126.7) (size 0.55) (drill 0.25) (layers "F.Cu" "B.Cu") (free) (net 2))
 (via (at 132.8 107.55) (size 0.55) (drill 0.25) (layers "F.Cu" "B.Cu") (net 2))
 (via (at 127.5 123.2) (size 0.55) (drill 0.25) (layers "F.Cu" "B.Cu") (free) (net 2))
 (via (at 126.8 122.5) (size 0.55) (drill 0.25) (layers "F.Cu" "B.Cu") (free) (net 2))
 (via (at 115.3 126) (size 0.55) (drill 0.25) (layers "F.Cu" "B.Cu") (free) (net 2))
 (via (at 112.4 122.5) (size 0.55) (drill 0.25) (layers "F.Cu" "B.Cu") (free) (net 2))
 (via (at 127.5 122.5) (size 0.55) (drill 0.25) (layers "F.Cu" "B.Cu") (free) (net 2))
 (via (at 124.6 122.5) (size 0.55) (drill 0.25) (layers "F.Cu" "B.Cu") (free) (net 2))
 (via (at 115.3 123.9) (size 0.55) (drill 0.25) (layers "F.Cu" "B.Cu") (free) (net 2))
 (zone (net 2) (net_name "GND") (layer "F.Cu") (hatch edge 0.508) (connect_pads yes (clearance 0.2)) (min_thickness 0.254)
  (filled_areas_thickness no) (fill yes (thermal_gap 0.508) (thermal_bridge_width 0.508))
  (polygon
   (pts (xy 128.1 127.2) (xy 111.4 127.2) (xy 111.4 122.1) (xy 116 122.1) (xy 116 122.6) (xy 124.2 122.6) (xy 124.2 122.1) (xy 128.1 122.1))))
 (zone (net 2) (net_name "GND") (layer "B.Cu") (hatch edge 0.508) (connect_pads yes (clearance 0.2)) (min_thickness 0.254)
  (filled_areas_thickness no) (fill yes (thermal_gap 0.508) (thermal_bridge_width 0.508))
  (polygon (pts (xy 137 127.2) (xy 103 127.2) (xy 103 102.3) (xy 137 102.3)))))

